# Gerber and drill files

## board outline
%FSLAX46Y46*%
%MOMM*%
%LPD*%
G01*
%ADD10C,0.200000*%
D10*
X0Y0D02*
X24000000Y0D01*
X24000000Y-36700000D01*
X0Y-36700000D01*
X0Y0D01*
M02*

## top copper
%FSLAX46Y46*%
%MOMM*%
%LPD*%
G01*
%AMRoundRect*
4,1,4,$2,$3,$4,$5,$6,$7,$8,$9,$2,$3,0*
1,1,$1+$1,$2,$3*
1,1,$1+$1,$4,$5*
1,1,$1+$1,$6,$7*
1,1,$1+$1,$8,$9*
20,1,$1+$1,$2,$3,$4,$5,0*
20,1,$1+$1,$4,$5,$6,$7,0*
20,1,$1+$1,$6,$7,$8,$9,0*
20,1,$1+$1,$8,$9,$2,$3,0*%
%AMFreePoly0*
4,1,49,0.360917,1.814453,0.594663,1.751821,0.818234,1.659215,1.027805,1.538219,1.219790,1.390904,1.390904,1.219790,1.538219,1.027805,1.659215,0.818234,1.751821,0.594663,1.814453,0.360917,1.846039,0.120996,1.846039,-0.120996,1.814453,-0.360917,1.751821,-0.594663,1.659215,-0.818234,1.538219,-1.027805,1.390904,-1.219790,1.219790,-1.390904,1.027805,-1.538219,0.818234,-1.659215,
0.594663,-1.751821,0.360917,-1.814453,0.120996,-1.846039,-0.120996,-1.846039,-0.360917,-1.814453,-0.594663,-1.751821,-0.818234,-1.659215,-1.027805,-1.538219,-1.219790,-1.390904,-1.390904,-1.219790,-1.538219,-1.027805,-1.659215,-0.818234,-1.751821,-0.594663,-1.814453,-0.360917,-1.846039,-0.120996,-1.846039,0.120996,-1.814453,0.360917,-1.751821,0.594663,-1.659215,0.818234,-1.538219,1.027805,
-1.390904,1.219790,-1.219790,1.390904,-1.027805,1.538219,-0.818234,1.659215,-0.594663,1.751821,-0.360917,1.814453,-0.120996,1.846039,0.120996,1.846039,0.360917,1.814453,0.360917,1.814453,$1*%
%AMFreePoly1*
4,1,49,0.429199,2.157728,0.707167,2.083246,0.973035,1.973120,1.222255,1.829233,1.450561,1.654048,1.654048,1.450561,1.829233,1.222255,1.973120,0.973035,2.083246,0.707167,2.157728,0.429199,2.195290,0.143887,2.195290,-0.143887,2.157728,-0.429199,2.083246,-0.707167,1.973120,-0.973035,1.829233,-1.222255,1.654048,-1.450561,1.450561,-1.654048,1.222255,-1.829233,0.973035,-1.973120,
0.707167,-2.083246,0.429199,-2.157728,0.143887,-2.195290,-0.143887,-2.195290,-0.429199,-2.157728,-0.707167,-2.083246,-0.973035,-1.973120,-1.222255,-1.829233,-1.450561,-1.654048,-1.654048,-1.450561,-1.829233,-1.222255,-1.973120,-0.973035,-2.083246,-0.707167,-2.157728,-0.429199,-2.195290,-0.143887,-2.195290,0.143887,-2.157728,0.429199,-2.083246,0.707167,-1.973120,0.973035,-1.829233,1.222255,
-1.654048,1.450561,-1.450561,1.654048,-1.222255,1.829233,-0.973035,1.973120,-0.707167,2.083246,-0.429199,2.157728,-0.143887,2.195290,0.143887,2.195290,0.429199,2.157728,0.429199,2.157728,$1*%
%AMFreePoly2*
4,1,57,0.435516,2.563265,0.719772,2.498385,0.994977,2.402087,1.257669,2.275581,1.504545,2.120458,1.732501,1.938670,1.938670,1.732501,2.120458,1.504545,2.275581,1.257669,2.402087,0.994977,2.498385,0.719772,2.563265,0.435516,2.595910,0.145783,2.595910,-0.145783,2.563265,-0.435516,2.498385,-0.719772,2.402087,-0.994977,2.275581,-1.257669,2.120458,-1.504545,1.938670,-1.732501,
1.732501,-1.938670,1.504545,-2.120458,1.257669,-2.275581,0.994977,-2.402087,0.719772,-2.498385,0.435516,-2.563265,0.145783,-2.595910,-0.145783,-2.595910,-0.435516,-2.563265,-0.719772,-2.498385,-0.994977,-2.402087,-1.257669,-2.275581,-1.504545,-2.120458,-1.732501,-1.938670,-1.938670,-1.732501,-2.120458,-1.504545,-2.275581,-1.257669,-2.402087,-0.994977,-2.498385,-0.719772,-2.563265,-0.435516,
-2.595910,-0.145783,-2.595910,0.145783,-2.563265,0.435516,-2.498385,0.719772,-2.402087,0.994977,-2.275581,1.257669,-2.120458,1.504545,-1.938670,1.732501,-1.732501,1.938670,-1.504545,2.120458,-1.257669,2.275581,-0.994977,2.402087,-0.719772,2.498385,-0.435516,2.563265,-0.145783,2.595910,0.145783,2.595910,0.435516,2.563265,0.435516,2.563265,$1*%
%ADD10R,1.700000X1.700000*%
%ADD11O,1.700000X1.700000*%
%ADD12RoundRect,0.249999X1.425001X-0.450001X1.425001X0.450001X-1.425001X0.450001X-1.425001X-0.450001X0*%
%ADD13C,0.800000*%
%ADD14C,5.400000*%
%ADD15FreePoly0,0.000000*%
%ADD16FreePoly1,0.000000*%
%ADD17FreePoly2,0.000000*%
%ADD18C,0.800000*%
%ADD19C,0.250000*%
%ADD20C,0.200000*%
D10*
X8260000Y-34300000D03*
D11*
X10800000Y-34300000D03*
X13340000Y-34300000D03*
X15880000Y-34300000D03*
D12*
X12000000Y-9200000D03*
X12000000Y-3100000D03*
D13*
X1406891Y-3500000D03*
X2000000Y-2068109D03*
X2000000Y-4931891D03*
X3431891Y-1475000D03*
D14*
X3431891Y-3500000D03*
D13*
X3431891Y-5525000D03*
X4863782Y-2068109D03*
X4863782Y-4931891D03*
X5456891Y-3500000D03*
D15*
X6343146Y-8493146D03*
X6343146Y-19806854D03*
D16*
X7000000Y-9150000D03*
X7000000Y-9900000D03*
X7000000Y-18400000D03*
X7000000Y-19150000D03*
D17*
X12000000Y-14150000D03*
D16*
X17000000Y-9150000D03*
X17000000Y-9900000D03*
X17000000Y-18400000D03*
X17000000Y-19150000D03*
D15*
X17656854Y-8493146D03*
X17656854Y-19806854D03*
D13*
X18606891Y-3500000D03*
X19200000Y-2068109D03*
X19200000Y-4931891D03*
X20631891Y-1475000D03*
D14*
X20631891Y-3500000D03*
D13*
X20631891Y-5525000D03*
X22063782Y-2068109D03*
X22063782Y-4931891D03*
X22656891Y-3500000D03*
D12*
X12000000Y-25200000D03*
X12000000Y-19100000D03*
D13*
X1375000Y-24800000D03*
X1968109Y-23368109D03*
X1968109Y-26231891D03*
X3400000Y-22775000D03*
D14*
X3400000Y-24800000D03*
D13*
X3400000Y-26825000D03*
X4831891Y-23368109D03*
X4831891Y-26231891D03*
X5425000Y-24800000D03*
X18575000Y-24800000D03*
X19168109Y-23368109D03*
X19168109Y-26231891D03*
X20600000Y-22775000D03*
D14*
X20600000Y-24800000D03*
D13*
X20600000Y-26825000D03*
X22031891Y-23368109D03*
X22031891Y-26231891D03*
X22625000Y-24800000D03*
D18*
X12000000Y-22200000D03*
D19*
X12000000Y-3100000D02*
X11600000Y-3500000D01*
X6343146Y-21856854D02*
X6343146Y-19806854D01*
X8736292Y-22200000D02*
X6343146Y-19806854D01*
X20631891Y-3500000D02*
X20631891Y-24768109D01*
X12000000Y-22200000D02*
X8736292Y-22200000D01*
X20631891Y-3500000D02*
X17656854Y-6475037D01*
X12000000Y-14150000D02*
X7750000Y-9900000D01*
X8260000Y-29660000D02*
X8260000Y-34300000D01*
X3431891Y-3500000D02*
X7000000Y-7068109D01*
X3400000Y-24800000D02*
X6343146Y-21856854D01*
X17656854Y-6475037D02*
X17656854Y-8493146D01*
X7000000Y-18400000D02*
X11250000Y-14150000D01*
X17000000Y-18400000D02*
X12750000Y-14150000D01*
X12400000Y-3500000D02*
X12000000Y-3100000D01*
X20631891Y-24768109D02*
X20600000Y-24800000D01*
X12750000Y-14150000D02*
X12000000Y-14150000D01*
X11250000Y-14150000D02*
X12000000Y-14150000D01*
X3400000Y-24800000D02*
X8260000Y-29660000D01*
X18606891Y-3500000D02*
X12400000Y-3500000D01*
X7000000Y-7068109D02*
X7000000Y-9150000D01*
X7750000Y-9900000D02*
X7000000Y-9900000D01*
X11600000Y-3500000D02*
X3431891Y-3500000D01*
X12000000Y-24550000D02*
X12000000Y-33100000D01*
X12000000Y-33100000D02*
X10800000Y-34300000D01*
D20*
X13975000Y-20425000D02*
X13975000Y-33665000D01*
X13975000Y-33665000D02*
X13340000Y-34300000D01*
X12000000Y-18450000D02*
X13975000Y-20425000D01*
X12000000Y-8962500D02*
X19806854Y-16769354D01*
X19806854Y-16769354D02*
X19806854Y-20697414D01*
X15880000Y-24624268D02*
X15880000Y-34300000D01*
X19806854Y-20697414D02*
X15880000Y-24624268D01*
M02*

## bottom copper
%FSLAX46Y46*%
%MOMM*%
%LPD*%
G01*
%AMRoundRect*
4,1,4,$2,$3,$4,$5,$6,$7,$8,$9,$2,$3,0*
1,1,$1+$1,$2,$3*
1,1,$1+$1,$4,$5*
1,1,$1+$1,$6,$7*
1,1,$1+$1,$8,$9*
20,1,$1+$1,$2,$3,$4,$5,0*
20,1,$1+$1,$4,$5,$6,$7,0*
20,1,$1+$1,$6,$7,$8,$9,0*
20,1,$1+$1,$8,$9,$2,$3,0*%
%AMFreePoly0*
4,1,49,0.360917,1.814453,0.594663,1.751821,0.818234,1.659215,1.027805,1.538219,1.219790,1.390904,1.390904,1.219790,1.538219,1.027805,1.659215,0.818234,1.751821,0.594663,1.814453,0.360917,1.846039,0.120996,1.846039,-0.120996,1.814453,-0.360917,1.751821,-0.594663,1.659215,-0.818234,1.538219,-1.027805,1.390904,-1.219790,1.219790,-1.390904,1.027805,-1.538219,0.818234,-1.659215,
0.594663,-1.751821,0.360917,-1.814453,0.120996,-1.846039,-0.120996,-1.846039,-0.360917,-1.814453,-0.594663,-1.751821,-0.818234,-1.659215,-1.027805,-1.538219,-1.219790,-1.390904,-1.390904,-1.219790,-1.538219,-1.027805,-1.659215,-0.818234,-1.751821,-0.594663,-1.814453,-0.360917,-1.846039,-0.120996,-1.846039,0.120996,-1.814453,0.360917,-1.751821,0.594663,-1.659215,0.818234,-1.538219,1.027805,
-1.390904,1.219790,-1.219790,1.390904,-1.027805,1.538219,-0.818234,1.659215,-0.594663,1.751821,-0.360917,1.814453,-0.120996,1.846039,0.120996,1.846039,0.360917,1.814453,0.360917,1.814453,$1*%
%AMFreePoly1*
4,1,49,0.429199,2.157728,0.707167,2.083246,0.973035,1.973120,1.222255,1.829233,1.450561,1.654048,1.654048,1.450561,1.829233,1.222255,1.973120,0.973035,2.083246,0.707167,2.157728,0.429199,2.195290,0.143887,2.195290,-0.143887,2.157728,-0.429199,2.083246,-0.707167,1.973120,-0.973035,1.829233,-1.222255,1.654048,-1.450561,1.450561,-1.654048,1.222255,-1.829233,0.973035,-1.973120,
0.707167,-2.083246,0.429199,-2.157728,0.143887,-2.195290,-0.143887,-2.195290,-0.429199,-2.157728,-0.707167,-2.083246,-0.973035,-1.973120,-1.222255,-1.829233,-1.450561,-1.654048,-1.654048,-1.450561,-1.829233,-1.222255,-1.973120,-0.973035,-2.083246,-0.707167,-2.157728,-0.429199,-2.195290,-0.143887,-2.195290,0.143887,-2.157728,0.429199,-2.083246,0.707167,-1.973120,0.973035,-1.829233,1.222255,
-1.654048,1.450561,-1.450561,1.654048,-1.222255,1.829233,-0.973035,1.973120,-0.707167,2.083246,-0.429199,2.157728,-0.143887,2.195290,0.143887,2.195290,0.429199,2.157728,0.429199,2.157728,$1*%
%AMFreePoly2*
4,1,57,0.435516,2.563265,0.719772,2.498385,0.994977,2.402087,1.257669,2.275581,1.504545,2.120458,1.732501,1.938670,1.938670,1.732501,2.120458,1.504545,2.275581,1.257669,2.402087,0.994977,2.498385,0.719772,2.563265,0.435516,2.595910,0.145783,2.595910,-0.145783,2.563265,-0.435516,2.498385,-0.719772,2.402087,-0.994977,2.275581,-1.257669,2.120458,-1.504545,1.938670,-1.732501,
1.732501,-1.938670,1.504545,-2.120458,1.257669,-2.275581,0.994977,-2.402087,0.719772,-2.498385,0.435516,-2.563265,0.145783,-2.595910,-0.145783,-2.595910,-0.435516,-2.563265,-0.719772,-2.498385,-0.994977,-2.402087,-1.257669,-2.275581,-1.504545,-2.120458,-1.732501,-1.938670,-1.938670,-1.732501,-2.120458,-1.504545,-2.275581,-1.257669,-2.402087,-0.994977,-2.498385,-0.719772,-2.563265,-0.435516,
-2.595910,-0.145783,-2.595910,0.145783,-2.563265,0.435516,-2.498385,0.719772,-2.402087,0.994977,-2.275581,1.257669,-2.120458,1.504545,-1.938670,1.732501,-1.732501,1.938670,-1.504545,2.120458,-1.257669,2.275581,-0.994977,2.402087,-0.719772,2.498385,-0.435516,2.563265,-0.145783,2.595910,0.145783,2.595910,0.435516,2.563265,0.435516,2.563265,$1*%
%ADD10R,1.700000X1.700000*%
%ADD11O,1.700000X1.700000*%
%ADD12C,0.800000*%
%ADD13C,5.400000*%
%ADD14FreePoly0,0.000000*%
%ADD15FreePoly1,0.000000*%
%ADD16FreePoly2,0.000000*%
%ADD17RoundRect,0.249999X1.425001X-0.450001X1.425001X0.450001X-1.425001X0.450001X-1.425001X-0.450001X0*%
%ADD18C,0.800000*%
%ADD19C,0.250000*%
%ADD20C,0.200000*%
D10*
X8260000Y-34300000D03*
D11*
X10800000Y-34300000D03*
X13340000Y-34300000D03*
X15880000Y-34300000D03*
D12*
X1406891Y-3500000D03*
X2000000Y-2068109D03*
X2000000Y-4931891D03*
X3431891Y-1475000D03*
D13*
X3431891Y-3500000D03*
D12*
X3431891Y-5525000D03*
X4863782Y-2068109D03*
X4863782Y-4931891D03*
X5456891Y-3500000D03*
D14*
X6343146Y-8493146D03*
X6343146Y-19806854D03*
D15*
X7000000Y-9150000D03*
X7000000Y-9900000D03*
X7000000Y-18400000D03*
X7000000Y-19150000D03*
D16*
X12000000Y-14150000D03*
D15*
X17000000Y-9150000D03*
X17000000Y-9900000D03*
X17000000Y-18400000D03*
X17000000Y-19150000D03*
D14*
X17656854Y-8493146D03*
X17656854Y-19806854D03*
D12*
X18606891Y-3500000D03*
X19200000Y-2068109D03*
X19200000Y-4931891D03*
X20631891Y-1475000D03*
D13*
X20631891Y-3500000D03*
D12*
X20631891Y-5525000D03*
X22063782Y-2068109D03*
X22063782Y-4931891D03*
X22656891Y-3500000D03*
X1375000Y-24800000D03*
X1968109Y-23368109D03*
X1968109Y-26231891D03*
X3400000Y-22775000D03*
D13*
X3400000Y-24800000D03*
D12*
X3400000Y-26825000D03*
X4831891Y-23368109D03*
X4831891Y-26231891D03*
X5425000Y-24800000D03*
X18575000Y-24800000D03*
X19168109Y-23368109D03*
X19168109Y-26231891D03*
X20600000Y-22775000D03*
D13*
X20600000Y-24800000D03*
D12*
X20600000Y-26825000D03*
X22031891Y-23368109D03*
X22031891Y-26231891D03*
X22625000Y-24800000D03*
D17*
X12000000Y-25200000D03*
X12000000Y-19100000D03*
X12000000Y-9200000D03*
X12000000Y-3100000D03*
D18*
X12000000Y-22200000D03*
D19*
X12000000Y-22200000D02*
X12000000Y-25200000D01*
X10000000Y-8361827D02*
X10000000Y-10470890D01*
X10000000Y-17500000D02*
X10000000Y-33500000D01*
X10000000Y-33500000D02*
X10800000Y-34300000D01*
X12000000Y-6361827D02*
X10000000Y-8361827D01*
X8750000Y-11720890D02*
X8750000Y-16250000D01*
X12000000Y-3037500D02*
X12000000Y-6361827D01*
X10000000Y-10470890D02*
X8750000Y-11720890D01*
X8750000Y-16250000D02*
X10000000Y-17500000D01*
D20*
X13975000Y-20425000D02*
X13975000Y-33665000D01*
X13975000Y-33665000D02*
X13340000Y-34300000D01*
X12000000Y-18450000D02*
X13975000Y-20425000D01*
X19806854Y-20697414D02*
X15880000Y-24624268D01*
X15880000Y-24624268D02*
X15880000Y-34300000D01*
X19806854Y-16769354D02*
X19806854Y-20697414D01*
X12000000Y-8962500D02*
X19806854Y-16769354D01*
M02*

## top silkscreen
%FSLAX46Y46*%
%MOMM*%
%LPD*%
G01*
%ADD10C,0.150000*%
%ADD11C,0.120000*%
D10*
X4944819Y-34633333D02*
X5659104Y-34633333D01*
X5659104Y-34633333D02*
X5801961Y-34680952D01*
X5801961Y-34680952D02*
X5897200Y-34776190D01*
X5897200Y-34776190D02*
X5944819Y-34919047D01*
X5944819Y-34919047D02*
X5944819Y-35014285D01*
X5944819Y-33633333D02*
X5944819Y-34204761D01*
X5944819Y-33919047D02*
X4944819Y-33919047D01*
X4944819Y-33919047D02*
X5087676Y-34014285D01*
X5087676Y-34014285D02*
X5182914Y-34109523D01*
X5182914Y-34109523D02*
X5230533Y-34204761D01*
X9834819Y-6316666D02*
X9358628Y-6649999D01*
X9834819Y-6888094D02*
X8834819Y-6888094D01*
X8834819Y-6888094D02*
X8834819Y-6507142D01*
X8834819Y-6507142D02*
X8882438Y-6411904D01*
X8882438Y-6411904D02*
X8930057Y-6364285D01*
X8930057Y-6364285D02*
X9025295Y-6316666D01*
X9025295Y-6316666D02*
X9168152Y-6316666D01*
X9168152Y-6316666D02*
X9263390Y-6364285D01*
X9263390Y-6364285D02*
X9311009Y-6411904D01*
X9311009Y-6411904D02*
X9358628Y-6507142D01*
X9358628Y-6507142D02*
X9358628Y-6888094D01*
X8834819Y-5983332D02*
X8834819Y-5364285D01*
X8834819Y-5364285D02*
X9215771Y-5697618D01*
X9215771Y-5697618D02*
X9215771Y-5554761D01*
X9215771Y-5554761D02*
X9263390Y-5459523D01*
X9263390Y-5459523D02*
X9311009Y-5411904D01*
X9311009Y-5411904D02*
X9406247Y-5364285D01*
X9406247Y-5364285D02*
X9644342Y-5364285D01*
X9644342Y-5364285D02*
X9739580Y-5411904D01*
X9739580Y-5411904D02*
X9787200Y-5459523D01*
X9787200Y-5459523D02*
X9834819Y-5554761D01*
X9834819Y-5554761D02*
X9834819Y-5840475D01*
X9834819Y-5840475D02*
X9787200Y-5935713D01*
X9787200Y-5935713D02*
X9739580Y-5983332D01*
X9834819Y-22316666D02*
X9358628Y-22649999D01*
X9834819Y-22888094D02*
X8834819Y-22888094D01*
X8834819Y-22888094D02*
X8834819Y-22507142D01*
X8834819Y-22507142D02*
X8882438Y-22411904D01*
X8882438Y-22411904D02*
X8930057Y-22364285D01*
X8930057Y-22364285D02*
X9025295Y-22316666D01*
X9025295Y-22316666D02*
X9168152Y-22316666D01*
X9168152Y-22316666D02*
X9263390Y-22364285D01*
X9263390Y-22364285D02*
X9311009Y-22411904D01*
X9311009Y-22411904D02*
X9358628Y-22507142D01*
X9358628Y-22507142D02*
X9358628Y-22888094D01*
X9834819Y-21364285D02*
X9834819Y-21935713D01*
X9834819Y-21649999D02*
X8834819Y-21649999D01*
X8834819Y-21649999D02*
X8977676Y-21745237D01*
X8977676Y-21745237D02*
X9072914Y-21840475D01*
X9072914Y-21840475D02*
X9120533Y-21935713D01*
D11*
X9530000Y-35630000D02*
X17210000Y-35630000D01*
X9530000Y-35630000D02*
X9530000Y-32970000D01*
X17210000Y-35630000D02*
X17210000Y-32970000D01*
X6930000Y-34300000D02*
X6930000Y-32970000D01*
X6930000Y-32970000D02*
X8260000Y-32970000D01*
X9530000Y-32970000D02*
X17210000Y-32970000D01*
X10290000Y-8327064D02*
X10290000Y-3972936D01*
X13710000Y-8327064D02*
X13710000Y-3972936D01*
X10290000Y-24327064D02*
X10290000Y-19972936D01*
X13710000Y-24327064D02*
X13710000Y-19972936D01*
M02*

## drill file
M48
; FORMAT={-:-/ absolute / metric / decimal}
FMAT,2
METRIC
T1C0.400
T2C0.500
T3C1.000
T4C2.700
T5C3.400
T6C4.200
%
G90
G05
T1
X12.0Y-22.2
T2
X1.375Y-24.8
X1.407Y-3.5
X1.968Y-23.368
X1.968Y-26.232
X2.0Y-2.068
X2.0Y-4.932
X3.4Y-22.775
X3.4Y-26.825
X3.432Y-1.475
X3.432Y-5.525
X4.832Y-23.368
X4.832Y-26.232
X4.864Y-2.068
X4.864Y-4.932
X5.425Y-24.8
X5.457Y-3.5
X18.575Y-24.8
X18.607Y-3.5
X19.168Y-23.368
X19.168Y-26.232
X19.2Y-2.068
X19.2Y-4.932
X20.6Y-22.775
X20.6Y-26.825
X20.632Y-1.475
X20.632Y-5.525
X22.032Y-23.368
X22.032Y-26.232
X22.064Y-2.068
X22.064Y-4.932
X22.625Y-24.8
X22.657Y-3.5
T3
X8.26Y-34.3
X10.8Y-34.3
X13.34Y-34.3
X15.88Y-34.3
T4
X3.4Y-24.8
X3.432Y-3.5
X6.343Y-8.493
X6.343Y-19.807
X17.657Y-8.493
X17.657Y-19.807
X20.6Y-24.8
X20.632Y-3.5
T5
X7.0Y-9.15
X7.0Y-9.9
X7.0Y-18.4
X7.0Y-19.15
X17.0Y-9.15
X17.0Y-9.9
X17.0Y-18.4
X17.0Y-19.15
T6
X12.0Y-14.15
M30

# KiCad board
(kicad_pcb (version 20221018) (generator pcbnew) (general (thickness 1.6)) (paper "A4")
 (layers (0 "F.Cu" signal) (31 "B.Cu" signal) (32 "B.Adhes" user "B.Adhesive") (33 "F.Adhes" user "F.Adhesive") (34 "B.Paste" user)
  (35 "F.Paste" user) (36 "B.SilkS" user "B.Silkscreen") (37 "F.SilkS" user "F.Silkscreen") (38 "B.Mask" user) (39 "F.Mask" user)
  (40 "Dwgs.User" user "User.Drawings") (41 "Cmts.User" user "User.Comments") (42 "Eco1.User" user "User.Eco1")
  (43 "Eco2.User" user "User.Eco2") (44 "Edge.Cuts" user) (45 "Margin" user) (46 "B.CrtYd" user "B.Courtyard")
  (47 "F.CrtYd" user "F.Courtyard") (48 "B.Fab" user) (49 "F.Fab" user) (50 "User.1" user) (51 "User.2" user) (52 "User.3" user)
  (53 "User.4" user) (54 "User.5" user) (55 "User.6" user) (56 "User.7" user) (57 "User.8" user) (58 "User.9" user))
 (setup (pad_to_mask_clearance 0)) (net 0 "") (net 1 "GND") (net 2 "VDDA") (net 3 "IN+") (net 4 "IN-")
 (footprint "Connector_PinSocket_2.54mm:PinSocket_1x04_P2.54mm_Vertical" (layer "F.Cu") (at 8.26 34.3 90)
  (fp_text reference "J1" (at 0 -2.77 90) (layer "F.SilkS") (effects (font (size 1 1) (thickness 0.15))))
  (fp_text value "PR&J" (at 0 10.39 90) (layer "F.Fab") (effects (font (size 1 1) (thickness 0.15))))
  (fp_line (start -1.33 1.27) (end -1.33 8.95) (stroke (width 0.12) (type solid)) (layer "F.SilkS"))
  (fp_line (start -1.33 1.27) (end 1.33 1.27) (stroke (width 0.12) (type solid)) (layer "F.SilkS"))
  (fp_line (start -1.33 8.95) (end 1.33 8.95) (stroke (width 0.12) (type solid)) (layer "F.SilkS"))
  (fp_line (start 0 -1.33) (end 1.33 -1.33) (stroke (width 0.12) (type solid)) (layer "F.SilkS"))
  (fp_line (start 1.33 -1.33) (end 1.33 0) (stroke (width 0.12) (type solid)) (layer "F.SilkS"))
  (fp_line (start 1.33 1.27) (end 1.33 8.95) (stroke (width 0.12) (type solid)) (layer "F.SilkS"))
  (pad "1" thru_hole rect (at 0 0 90) (size 1.7 1.7) (drill 1) (layers "*.Cu" "*.Mask") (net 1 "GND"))
  (pad "2" thru_hole oval (at 0 2.54 90) (size 1.7 1.7) (drill 1) (layers "*.Cu" "*.Mask") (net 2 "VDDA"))
  (pad "3" thru_hole oval (at 0 5.08 90) (size 1.7 1.7) (drill 1) (layers "*.Cu" "*.Mask") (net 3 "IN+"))
  (pad "4" thru_hole oval (at 0 7.62 90) (size 1.7 1.7) (drill 1) (layers "*.Cu" "*.Mask") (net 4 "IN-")))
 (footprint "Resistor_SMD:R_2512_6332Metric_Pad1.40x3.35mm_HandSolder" (layer "F.Cu") (at 12 6.15 90)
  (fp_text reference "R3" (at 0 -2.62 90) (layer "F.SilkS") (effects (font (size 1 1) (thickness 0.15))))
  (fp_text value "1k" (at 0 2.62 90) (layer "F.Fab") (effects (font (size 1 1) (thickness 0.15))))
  (fp_line (start -2.177064 -1.71) (end 2.177064 -1.71) (stroke (width 0.12) (type solid)) (layer "F.SilkS"))
  (fp_line (start -2.177064 1.71) (end 2.177064 1.71) (stroke (width 0.12) (type solid)) (layer "F.SilkS"))
  (pad "1" smd roundrect (at -3.05 0 90) (size 1.4 3.35) (layers "F.Cu" "F.Paste" "F.Mask") (roundrect_rratio 0.1785707143) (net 4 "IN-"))
  (pad "2" smd roundrect (at 3.05 0 90) (size 1.4 3.35) (layers "F.Cu" "F.Paste" "F.Mask") (roundrect_rratio 0.1785707143) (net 1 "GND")))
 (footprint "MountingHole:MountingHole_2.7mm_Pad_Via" (layer "F.Cu") (at 3.431891 3.5)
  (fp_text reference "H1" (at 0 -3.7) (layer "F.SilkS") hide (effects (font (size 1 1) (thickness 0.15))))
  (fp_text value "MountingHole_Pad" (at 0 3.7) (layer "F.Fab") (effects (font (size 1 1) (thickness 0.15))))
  (pad "1" thru_hole circle (at -2.025 0) (size 0.8 0.8) (drill 0.5) (layers "*.Cu" "*.Mask") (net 1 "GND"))
  (pad "1" thru_hole circle (at -1.431891 -1.431891) (size 0.8 0.8) (drill 0.5) (layers "*.Cu" "*.Mask") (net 1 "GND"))
  (pad "1" thru_hole circle (at -1.431891 1.431891) (size 0.8 0.8) (drill 0.5) (layers "*.Cu" "*.Mask") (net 1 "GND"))
  (pad "1" thru_hole circle (at 0 -2.025) (size 0.8 0.8) (drill 0.5) (layers "*.Cu" "*.Mask") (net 1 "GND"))
  (pad "1" thru_hole circle (at 0 0) (size 5.4 5.4) (drill 2.7) (layers "*.Cu" "*.Mask") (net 1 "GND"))
  (pad "1" thru_hole circle (at 0 2.025) (size 0.8 0.8) (drill 0.5) (layers "*.Cu" "*.Mask") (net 1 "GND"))
  (pad "1" thru_hole circle (at 1.431891 -1.431891) (size 0.8 0.8) (drill 0.5) (layers "*.Cu" "*.Mask") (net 1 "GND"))
  (pad "1" thru_hole circle (at 1.431891 1.431891) (size 0.8 0.8) (drill 0.5) (layers "*.Cu" "*.Mask") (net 1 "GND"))
  (pad "1" thru_hole circle (at 2.025 0) (size 0.8 0.8) (drill 0.5) (layers "*.Cu" "*.Mask") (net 1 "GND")))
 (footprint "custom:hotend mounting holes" (layer "F.Cu") (at 12 14.15)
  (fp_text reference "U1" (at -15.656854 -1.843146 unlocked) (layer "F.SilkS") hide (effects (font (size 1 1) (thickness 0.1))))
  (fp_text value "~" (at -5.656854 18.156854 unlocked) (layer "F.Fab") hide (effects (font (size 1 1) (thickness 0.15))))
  (pad "1" thru_hole custom (at -5.656854 -5.656854) (size 3.7 3.7) (drill 2.7) (layers "*.Cu" "*.Mask") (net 1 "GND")
   (thermal_bridge_angle 45) (options (clearance outline) (anchor circle)) (primitives))
  (pad "1" thru_hole custom (at -5.656854 5.656854) (size 3.7 3.7) (drill 2.7) (layers "*.Cu" "*.Mask") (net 1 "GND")
   (thermal_bridge_angle 45) (options (clearance outline) (anchor circle)) (primitives))
  (pad "1" thru_hole custom (at -5 -5) (size 4.4 4.4) (drill 3.4) (layers "*.Cu" "*.Mask") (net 1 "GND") (thermal_bridge_angle 45)
   (options (clearance outline) (anchor circle)) (primitives))
  (pad "1" thru_hole custom (at -5 -4.25) (size 4.4 4.4) (drill 3.4) (layers "*.Cu" "*.Mask") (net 1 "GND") (thermal_bridge_angle 45)
   (options (clearance outline) (anchor circle)) (primitives))
  (pad "1" thru_hole custom (at -5 4.25) (size 4.4 4.4) (drill 3.4) (layers "*.Cu" "*.Mask") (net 1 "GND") (thermal_bridge_angle 45)
   (options (clearance outline) (anchor circle)) (primitives))
  (pad "1" thru_hole custom (at -5 5) (size 4.4 4.4) (drill 3.4) (layers "*.Cu" "*.Mask") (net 1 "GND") (thermal_bridge_angle 45)
   (options (clearance outline) (anchor circle)) (primitives))
  (pad "1" thru_hole custom (at 0 0) (size 5.2 5.2) (drill 4.2) (layers "*.Cu" "*.Mask") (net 1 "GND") (thermal_bridge_angle 45)
   (options (clearance outline) (anchor circle)) (primitives))
  (pad "1" thru_hole custom (at 5 -5) (size 4.4 4.4) (drill 3.4) (layers "*.Cu" "*.Mask") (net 1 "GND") (thermal_bridge_angle 45)
   (options (clearance outline) (anchor circle)) (primitives))
  (pad "1" thru_hole custom (at 5 -4.25) (size 4.4 4.4) (drill 3.4) (layers "*.Cu" "*.Mask") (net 1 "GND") (thermal_bridge_angle 45)
   (options (clearance outline) (anchor circle)) (primitives))
  (pad "1" thru_hole custom (at 5 4.25) (size 4.4 4.4) (drill 3.4) (layers "*.Cu" "*.Mask") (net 1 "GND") (thermal_bridge_angle 45)
   (options (clearance outline) (anchor circle)) (primitives))
  (pad "1" thru_hole custom (at 5 5) (size 4.4 4.4) (drill 3.4) (layers "*.Cu" "*.Mask") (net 1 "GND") (thermal_bridge_angle 45)
   (options (clearance outline) (anchor circle)) (primitives))
  (pad "1" thru_hole custom (at 5.656854 -5.656854) (size 3.7 3.7) (drill 2.7) (layers "*.Cu" "*.Mask") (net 1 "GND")
   (thermal_bridge_angle 45) (options (clearance outline) (anchor circle)) (primitives))
  (pad "1" thru_hole custom (at 5.656854 5.656854) (size 3.7 3.7) (drill 2.7) (layers "*.Cu" "*.Mask") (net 1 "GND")
   (thermal_bridge_angle 45) (options (clearance outline) (anchor circle)) (primitives)))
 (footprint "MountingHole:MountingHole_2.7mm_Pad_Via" (layer "F.Cu") (at 20.631891 3.5)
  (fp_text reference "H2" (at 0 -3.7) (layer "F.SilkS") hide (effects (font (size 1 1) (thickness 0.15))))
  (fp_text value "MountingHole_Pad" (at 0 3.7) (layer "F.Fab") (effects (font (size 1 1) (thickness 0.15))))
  (pad "1" thru_hole circle (at -2.025 0) (size 0.8 0.8) (drill 0.5) (layers "*.Cu" "*.Mask") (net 1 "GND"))
  (pad "1" thru_hole circle (at -1.431891 -1.431891) (size 0.8 0.8) (drill 0.5) (layers "*.Cu" "*.Mask") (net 1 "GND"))
  (pad "1" thru_hole circle (at -1.431891 1.431891) (size 0.8 0.8) (drill 0.5) (layers "*.Cu" "*.Mask") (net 1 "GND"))
  (pad "1" thru_hole circle (at 0 -2.025) (size 0.8 0.8) (drill 0.5) (layers "*.Cu" "*.Mask") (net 1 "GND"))
  (pad "1" thru_hole circle (at 0 0) (size 5.4 5.4) (drill 2.7) (layers "*.Cu" "*.Mask") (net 1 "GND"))
  (pad "1" thru_hole circle (at 0 2.025) (size 0.8 0.8) (drill 0.5) (layers "*.Cu" "*.Mask") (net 1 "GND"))
  (pad "1" thru_hole circle (at 1.431891 -1.431891) (size 0.8 0.8) (drill 0.5) (layers "*.Cu" "*.Mask") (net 1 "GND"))
  (pad "1" thru_hole circle (at 1.431891 1.431891) (size 0.8 0.8) (drill 0.5) (layers "*.Cu" "*.Mask") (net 1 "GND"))
  (pad "1" thru_hole circle (at 2.025 0) (size 0.8 0.8) (drill 0.5) (layers "*.Cu" "*.Mask") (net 1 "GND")))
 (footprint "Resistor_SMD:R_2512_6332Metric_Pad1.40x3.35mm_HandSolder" (layer "F.Cu") (at 12 22.15 90)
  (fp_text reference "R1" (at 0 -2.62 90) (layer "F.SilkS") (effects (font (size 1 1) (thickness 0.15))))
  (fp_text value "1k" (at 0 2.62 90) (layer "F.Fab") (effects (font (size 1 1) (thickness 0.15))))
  (fp_line (start -2.177064 -1.71) (end 2.177064 -1.71) (stroke (width 0.12) (type solid)) (layer "F.SilkS"))
  (fp_line (start -2.177064 1.71) (end 2.177064 1.71) (stroke (width 0.12) (type solid)) (layer "F.SilkS"))
  (pad "1" smd roundrect (at -3.05 0 90) (size 1.4 3.35) (layers "F.Cu" "F.Paste" "F.Mask") (roundrect_rratio 0.1785707143) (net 2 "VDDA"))
  (pad "2" smd roundrect (at 3.05 0 90) (size 1.4 3.35) (layers "F.Cu" "F.Paste" "F.Mask") (roundrect_rratio 0.1785707143) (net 3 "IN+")))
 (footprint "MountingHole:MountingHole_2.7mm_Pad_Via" (layer "F.Cu") (at 3.4 24.8)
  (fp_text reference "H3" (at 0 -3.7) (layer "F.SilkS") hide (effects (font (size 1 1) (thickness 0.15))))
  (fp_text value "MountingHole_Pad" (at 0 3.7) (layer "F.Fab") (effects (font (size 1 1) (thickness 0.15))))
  (pad "1" thru_hole circle (at -2.025 0) (size 0.8 0.8) (drill 0.5) (layers "*.Cu" "*.Mask") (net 1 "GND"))
  (pad "1" thru_hole circle (at -1.431891 -1.431891) (size 0.8 0.8) (drill 0.5) (layers "*.Cu" "*.Mask") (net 1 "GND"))
  (pad "1" thru_hole circle (at -1.431891 1.431891) (size 0.8 0.8) (drill 0.5) (layers "*.Cu" "*.Mask") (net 1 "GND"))
  (pad "1" thru_hole circle (at 0 -2.025) (size 0.8 0.8) (drill 0.5) (layers "*.Cu" "*.Mask") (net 1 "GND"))
  (pad "1" thru_hole circle (at 0 0) (size 5.4 5.4) (drill 2.7) (layers "*.Cu" "*.Mask") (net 1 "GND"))
  (pad "1" thru_hole circle (at 0 2.025) (size 0.8 0.8) (drill 0.5) (layers "*.Cu" "*.Mask") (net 1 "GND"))
  (pad "1" thru_hole circle (at 1.431891 -1.431891) (size 0.8 0.8) (drill 0.5) (layers "*.Cu" "*.Mask") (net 1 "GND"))
  (pad "1" thru_hole circle (at 1.431891 1.431891) (size 0.8 0.8) (drill 0.5) (layers "*.Cu" "*.Mask") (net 1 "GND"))
  (pad "1" thru_hole circle (at 2.025 0) (size 0.8 0.8) (drill 0.5) (layers "*.Cu" "*.Mask") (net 1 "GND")))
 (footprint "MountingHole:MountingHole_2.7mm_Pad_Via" (layer "F.Cu") (at 20.6 24.8)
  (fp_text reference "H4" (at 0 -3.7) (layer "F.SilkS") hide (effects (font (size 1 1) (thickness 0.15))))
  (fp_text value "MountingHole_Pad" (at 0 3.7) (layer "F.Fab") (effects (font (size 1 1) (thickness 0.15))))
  (pad "1" thru_hole circle (at -2.025 0) (size 0.8 0.8) (drill 0.5) (layers "*.Cu" "*.Mask") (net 1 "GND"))
  (pad "1" thru_hole circle (at -1.431891 -1.431891) (size 0.8 0.8) (drill 0.5) (layers "*.Cu" "*.Mask") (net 1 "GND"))
  (pad "1" thru_hole circle (at -1.431891 1.431891) (size 0.8 0.8) (drill 0.5) (layers "*.Cu" "*.Mask") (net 1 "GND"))
  (pad "1" thru_hole circle (at 0 -2.025) (size 0.8 0.8) (drill 0.5) (layers "*.Cu" "*.Mask") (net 1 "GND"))
  (pad "1" thru_hole circle (at 0 0) (size 5.4 5.4) (drill 2.7) (layers "*.Cu" "*.Mask") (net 1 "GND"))
  (pad "1" thru_hole circle (at 0 2.025) (size 0.8 0.8) (drill 0.5) (layers "*.Cu" "*.Mask") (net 1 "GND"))
  (pad "1" thru_hole circle (at 1.431891 -1.431891) (size 0.8 0.8) (drill 0.5) (layers "*.Cu" "*.Mask") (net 1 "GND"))
  (pad "1" thru_hole circle (at 1.431891 1.431891) (size 0.8 0.8) (drill 0.5) (layers "*.Cu" "*.Mask") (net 1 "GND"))
  (pad "1" thru_hole circle (at 2.025 0) (size 0.8 0.8) (drill 0.5) (layers "*.Cu" "*.Mask") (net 1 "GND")))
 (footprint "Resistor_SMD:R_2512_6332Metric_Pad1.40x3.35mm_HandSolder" (layer "B.Cu") (at 12 22.15 90)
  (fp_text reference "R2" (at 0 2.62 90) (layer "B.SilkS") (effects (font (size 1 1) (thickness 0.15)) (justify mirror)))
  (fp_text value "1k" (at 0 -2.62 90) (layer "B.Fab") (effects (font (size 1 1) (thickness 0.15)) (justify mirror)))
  (pad "1" smd roundrect (at -3.05 0 90) (size 1.4 3.35) (layers "B.Cu" "B.Paste" "B.Mask") (roundrect_rratio 0.1785707143) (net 1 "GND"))
  (pad "2" smd roundrect (at 3.05 0 90) (size 1.4 3.35) (layers "B.Cu" "B.Paste" "B.Mask") (roundrect_rratio 0.1785707143) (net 3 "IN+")))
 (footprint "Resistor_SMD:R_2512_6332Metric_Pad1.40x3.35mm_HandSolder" (layer "B.Cu") (at 12 6.15 90)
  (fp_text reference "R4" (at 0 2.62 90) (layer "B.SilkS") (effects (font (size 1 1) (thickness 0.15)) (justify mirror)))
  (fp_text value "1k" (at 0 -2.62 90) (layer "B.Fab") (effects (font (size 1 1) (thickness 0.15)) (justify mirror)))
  (pad "1" smd roundrect (at -3.05 0 90) (size 1.4 3.35) (layers "B.Cu" "B.Paste" "B.Mask") (roundrect_rratio 0.1785707143) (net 4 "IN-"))
  (pad "2" smd roundrect (at 3.05 0 90) (size 1.4 3.35) (layers "B.Cu" "B.Paste" "B.Mask") (roundrect_rratio 0.1785707143) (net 2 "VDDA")))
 (gr_rect (start 0 0) (end 24 36.7) (stroke (width 0.2) (type default)) (fill none) (layer "Edge.Cuts"))
 (segment (start 12 3.1) (end 11.6 3.5) (width 0.25) (layer "F.Cu") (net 1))
 (segment (start 6.343146 21.856854) (end 6.343146 19.806854) (width 0.25) (layer "F.Cu") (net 1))
 (segment (start 8.736292 22.2) (end 6.343146 19.806854) (width 0.25) (layer "F.Cu") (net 1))
 (segment (start 20.631891 3.5) (end 20.631891 24.768109) (width 0.25) (layer "F.Cu") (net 1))
 (segment (start 12 22.2) (end 8.736292 22.2) (width 0.25) (layer "F.Cu") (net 1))
 (segment (start 20.631891 3.5) (end 17.656854 6.475037) (width 0.25) (layer "F.Cu") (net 1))
 (segment (start 12 14.15) (end 7.75 9.9) (width 0.25) (layer "F.Cu") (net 1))
 (segment (start 8.26 29.66) (end 8.26 34.3) (width 0.25) (layer "F.Cu") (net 1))
 (segment (start 3.431891 3.5) (end 7 7.068109) (width 0.25) (layer "F.Cu") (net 1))
 (segment (start 3.4 24.8) (end 6.343146 21.856854) (width 0.25) (layer "F.Cu") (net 1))
 (segment (start 17.656854 6.475037) (end 17.656854 8.493146) (width 0.25) (layer "F.Cu") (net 1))
 (segment (start 7 18.4) (end 11.25 14.15) (width 0.25) (layer "F.Cu") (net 1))
 (segment (start 17 18.4) (end 12.75 14.15) (width 0.25) (layer "F.Cu") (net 1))
 (segment (start 12.4 3.5) (end 12 3.1) (width 0.25) (layer "F.Cu") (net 1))
 (segment (start 20.631891 24.768109) (end 20.6 24.8) (width 0.25) (layer "F.Cu") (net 1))
 (segment (start 12.75 14.15) (end 12 14.15) (width 0.25) (layer "F.Cu") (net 1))
 (segment (start 11.25 14.15) (end 12 14.15) (width 0.25) (layer "F.Cu") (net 1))
 (segment (start 3.4 24.8) (end 8.26 29.66) (width 0.25) (layer "F.Cu") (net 1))
 (segment (start 18.606891 3.5) (end 12.4 3.5) (width 0.25) (layer "F.Cu") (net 1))
 (segment (start 7 7.068109) (end 7 9.15) (width 0.25) (layer "F.Cu") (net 1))
 (segment (start 7.75 9.9) (end 7 9.9) (width 0.25) (layer "F.Cu") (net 1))
 (segment (start 11.6 3.5) (end 3.431891 3.5) (width 0.25) (layer "F.Cu") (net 1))
 (via (at 12 22.2) (size 0.8) (drill 0.4) (layers "F.Cu" "B.Cu") (free) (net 1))
 (segment (start 12 22.2) (end 12 25.2) (width 0.25) (layer "B.Cu") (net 1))
 (segment (start 12 24.55) (end 12 33.1) (width 0.25) (layer "F.Cu") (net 2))
 (segment (start 12 33.1) (end 10.8 34.3) (width 0.25) (layer "F.Cu") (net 2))
 (segment (start 10 8.361827) (end 10 10.47089) (width 0.25) (layer "B.Cu") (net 2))
 (segment (start 10 17.5) (end 10 33.5) (width 0.25) (layer "B.Cu") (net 2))
 (segment (start 10 33.5) (end 10.8 34.3) (width 0.25) (layer "B.Cu") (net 2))
 (segment (start 12 6.361827) (end 10 8.361827) (width 0.25) (layer "B.Cu") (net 2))
 (segment (start 8.75 11.72089) (end 8.75 16.25) (width 0.25) (layer "B.Cu") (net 2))
 (segment (start 12 3.0375) (end 12 6.361827) (width 0.25) (layer "B.Cu") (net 2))
 (segment (start 10 10.47089) (end 8.75 11.72089) (width 0.25) (layer "B.Cu") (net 2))
 (segment (start 8.75 16.25) (end 10 17.5) (width 0.25) (layer "B.Cu") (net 2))
 (segment (start 13.975 20.425) (end 13.975 33.665) (width 0.2) (layer "F.Cu") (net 3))
 (segment (start 13.975 33.665) (end 13.34 34.3) (width 0.2) (layer "F.Cu") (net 3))
 (segment (start 12 18.45) (end 13.975 20.425) (width 0.2) (layer "F.Cu") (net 3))
 (segment (start 13.975 20.425) (end 13.975 33.665) (width 0.2) (layer "B.Cu") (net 3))
 (segment (start 13.975 33.665) (end 13.34 34.3) (width 0.2) (layer "B.Cu") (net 3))
 (segment (start 12 18.45) (end 13.975 20.425) (width 0.2) (layer "B.Cu") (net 3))
 (segment (start 12 8.9625) (end 19.806854 16.769354) (width 0.2) (layer "F.Cu") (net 4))
 (segment (start 19.806854 16.769354) (end 19.806854 20.697414) (width 0.2) (layer "F.Cu") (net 4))
 (segment (start 15.88 24.624268) (end 15.88 34.3) (width 0.2) (layer "F.Cu") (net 4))
 (segment (start 19.806854 20.697414) (end 15.88 24.624268) (width 0.2) (layer "F.Cu") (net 4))
 (segment (start 19.806854 20.697414) (end 15.88 24.624268) (width 0.2) (layer "B.Cu") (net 4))
 (segment (start 15.88 24.624268) (end 15.88 34.3) (width 0.2) (layer "B.Cu") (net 4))
 (segment (start 19.806854 16.769354) (end 19.806854 20.697414) (width 0.2) (layer "B.Cu") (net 4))
 (segment (start 12 8.9625) (end 19.806854 16.769354) (width 0.2) (layer "B.Cu") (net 4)))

